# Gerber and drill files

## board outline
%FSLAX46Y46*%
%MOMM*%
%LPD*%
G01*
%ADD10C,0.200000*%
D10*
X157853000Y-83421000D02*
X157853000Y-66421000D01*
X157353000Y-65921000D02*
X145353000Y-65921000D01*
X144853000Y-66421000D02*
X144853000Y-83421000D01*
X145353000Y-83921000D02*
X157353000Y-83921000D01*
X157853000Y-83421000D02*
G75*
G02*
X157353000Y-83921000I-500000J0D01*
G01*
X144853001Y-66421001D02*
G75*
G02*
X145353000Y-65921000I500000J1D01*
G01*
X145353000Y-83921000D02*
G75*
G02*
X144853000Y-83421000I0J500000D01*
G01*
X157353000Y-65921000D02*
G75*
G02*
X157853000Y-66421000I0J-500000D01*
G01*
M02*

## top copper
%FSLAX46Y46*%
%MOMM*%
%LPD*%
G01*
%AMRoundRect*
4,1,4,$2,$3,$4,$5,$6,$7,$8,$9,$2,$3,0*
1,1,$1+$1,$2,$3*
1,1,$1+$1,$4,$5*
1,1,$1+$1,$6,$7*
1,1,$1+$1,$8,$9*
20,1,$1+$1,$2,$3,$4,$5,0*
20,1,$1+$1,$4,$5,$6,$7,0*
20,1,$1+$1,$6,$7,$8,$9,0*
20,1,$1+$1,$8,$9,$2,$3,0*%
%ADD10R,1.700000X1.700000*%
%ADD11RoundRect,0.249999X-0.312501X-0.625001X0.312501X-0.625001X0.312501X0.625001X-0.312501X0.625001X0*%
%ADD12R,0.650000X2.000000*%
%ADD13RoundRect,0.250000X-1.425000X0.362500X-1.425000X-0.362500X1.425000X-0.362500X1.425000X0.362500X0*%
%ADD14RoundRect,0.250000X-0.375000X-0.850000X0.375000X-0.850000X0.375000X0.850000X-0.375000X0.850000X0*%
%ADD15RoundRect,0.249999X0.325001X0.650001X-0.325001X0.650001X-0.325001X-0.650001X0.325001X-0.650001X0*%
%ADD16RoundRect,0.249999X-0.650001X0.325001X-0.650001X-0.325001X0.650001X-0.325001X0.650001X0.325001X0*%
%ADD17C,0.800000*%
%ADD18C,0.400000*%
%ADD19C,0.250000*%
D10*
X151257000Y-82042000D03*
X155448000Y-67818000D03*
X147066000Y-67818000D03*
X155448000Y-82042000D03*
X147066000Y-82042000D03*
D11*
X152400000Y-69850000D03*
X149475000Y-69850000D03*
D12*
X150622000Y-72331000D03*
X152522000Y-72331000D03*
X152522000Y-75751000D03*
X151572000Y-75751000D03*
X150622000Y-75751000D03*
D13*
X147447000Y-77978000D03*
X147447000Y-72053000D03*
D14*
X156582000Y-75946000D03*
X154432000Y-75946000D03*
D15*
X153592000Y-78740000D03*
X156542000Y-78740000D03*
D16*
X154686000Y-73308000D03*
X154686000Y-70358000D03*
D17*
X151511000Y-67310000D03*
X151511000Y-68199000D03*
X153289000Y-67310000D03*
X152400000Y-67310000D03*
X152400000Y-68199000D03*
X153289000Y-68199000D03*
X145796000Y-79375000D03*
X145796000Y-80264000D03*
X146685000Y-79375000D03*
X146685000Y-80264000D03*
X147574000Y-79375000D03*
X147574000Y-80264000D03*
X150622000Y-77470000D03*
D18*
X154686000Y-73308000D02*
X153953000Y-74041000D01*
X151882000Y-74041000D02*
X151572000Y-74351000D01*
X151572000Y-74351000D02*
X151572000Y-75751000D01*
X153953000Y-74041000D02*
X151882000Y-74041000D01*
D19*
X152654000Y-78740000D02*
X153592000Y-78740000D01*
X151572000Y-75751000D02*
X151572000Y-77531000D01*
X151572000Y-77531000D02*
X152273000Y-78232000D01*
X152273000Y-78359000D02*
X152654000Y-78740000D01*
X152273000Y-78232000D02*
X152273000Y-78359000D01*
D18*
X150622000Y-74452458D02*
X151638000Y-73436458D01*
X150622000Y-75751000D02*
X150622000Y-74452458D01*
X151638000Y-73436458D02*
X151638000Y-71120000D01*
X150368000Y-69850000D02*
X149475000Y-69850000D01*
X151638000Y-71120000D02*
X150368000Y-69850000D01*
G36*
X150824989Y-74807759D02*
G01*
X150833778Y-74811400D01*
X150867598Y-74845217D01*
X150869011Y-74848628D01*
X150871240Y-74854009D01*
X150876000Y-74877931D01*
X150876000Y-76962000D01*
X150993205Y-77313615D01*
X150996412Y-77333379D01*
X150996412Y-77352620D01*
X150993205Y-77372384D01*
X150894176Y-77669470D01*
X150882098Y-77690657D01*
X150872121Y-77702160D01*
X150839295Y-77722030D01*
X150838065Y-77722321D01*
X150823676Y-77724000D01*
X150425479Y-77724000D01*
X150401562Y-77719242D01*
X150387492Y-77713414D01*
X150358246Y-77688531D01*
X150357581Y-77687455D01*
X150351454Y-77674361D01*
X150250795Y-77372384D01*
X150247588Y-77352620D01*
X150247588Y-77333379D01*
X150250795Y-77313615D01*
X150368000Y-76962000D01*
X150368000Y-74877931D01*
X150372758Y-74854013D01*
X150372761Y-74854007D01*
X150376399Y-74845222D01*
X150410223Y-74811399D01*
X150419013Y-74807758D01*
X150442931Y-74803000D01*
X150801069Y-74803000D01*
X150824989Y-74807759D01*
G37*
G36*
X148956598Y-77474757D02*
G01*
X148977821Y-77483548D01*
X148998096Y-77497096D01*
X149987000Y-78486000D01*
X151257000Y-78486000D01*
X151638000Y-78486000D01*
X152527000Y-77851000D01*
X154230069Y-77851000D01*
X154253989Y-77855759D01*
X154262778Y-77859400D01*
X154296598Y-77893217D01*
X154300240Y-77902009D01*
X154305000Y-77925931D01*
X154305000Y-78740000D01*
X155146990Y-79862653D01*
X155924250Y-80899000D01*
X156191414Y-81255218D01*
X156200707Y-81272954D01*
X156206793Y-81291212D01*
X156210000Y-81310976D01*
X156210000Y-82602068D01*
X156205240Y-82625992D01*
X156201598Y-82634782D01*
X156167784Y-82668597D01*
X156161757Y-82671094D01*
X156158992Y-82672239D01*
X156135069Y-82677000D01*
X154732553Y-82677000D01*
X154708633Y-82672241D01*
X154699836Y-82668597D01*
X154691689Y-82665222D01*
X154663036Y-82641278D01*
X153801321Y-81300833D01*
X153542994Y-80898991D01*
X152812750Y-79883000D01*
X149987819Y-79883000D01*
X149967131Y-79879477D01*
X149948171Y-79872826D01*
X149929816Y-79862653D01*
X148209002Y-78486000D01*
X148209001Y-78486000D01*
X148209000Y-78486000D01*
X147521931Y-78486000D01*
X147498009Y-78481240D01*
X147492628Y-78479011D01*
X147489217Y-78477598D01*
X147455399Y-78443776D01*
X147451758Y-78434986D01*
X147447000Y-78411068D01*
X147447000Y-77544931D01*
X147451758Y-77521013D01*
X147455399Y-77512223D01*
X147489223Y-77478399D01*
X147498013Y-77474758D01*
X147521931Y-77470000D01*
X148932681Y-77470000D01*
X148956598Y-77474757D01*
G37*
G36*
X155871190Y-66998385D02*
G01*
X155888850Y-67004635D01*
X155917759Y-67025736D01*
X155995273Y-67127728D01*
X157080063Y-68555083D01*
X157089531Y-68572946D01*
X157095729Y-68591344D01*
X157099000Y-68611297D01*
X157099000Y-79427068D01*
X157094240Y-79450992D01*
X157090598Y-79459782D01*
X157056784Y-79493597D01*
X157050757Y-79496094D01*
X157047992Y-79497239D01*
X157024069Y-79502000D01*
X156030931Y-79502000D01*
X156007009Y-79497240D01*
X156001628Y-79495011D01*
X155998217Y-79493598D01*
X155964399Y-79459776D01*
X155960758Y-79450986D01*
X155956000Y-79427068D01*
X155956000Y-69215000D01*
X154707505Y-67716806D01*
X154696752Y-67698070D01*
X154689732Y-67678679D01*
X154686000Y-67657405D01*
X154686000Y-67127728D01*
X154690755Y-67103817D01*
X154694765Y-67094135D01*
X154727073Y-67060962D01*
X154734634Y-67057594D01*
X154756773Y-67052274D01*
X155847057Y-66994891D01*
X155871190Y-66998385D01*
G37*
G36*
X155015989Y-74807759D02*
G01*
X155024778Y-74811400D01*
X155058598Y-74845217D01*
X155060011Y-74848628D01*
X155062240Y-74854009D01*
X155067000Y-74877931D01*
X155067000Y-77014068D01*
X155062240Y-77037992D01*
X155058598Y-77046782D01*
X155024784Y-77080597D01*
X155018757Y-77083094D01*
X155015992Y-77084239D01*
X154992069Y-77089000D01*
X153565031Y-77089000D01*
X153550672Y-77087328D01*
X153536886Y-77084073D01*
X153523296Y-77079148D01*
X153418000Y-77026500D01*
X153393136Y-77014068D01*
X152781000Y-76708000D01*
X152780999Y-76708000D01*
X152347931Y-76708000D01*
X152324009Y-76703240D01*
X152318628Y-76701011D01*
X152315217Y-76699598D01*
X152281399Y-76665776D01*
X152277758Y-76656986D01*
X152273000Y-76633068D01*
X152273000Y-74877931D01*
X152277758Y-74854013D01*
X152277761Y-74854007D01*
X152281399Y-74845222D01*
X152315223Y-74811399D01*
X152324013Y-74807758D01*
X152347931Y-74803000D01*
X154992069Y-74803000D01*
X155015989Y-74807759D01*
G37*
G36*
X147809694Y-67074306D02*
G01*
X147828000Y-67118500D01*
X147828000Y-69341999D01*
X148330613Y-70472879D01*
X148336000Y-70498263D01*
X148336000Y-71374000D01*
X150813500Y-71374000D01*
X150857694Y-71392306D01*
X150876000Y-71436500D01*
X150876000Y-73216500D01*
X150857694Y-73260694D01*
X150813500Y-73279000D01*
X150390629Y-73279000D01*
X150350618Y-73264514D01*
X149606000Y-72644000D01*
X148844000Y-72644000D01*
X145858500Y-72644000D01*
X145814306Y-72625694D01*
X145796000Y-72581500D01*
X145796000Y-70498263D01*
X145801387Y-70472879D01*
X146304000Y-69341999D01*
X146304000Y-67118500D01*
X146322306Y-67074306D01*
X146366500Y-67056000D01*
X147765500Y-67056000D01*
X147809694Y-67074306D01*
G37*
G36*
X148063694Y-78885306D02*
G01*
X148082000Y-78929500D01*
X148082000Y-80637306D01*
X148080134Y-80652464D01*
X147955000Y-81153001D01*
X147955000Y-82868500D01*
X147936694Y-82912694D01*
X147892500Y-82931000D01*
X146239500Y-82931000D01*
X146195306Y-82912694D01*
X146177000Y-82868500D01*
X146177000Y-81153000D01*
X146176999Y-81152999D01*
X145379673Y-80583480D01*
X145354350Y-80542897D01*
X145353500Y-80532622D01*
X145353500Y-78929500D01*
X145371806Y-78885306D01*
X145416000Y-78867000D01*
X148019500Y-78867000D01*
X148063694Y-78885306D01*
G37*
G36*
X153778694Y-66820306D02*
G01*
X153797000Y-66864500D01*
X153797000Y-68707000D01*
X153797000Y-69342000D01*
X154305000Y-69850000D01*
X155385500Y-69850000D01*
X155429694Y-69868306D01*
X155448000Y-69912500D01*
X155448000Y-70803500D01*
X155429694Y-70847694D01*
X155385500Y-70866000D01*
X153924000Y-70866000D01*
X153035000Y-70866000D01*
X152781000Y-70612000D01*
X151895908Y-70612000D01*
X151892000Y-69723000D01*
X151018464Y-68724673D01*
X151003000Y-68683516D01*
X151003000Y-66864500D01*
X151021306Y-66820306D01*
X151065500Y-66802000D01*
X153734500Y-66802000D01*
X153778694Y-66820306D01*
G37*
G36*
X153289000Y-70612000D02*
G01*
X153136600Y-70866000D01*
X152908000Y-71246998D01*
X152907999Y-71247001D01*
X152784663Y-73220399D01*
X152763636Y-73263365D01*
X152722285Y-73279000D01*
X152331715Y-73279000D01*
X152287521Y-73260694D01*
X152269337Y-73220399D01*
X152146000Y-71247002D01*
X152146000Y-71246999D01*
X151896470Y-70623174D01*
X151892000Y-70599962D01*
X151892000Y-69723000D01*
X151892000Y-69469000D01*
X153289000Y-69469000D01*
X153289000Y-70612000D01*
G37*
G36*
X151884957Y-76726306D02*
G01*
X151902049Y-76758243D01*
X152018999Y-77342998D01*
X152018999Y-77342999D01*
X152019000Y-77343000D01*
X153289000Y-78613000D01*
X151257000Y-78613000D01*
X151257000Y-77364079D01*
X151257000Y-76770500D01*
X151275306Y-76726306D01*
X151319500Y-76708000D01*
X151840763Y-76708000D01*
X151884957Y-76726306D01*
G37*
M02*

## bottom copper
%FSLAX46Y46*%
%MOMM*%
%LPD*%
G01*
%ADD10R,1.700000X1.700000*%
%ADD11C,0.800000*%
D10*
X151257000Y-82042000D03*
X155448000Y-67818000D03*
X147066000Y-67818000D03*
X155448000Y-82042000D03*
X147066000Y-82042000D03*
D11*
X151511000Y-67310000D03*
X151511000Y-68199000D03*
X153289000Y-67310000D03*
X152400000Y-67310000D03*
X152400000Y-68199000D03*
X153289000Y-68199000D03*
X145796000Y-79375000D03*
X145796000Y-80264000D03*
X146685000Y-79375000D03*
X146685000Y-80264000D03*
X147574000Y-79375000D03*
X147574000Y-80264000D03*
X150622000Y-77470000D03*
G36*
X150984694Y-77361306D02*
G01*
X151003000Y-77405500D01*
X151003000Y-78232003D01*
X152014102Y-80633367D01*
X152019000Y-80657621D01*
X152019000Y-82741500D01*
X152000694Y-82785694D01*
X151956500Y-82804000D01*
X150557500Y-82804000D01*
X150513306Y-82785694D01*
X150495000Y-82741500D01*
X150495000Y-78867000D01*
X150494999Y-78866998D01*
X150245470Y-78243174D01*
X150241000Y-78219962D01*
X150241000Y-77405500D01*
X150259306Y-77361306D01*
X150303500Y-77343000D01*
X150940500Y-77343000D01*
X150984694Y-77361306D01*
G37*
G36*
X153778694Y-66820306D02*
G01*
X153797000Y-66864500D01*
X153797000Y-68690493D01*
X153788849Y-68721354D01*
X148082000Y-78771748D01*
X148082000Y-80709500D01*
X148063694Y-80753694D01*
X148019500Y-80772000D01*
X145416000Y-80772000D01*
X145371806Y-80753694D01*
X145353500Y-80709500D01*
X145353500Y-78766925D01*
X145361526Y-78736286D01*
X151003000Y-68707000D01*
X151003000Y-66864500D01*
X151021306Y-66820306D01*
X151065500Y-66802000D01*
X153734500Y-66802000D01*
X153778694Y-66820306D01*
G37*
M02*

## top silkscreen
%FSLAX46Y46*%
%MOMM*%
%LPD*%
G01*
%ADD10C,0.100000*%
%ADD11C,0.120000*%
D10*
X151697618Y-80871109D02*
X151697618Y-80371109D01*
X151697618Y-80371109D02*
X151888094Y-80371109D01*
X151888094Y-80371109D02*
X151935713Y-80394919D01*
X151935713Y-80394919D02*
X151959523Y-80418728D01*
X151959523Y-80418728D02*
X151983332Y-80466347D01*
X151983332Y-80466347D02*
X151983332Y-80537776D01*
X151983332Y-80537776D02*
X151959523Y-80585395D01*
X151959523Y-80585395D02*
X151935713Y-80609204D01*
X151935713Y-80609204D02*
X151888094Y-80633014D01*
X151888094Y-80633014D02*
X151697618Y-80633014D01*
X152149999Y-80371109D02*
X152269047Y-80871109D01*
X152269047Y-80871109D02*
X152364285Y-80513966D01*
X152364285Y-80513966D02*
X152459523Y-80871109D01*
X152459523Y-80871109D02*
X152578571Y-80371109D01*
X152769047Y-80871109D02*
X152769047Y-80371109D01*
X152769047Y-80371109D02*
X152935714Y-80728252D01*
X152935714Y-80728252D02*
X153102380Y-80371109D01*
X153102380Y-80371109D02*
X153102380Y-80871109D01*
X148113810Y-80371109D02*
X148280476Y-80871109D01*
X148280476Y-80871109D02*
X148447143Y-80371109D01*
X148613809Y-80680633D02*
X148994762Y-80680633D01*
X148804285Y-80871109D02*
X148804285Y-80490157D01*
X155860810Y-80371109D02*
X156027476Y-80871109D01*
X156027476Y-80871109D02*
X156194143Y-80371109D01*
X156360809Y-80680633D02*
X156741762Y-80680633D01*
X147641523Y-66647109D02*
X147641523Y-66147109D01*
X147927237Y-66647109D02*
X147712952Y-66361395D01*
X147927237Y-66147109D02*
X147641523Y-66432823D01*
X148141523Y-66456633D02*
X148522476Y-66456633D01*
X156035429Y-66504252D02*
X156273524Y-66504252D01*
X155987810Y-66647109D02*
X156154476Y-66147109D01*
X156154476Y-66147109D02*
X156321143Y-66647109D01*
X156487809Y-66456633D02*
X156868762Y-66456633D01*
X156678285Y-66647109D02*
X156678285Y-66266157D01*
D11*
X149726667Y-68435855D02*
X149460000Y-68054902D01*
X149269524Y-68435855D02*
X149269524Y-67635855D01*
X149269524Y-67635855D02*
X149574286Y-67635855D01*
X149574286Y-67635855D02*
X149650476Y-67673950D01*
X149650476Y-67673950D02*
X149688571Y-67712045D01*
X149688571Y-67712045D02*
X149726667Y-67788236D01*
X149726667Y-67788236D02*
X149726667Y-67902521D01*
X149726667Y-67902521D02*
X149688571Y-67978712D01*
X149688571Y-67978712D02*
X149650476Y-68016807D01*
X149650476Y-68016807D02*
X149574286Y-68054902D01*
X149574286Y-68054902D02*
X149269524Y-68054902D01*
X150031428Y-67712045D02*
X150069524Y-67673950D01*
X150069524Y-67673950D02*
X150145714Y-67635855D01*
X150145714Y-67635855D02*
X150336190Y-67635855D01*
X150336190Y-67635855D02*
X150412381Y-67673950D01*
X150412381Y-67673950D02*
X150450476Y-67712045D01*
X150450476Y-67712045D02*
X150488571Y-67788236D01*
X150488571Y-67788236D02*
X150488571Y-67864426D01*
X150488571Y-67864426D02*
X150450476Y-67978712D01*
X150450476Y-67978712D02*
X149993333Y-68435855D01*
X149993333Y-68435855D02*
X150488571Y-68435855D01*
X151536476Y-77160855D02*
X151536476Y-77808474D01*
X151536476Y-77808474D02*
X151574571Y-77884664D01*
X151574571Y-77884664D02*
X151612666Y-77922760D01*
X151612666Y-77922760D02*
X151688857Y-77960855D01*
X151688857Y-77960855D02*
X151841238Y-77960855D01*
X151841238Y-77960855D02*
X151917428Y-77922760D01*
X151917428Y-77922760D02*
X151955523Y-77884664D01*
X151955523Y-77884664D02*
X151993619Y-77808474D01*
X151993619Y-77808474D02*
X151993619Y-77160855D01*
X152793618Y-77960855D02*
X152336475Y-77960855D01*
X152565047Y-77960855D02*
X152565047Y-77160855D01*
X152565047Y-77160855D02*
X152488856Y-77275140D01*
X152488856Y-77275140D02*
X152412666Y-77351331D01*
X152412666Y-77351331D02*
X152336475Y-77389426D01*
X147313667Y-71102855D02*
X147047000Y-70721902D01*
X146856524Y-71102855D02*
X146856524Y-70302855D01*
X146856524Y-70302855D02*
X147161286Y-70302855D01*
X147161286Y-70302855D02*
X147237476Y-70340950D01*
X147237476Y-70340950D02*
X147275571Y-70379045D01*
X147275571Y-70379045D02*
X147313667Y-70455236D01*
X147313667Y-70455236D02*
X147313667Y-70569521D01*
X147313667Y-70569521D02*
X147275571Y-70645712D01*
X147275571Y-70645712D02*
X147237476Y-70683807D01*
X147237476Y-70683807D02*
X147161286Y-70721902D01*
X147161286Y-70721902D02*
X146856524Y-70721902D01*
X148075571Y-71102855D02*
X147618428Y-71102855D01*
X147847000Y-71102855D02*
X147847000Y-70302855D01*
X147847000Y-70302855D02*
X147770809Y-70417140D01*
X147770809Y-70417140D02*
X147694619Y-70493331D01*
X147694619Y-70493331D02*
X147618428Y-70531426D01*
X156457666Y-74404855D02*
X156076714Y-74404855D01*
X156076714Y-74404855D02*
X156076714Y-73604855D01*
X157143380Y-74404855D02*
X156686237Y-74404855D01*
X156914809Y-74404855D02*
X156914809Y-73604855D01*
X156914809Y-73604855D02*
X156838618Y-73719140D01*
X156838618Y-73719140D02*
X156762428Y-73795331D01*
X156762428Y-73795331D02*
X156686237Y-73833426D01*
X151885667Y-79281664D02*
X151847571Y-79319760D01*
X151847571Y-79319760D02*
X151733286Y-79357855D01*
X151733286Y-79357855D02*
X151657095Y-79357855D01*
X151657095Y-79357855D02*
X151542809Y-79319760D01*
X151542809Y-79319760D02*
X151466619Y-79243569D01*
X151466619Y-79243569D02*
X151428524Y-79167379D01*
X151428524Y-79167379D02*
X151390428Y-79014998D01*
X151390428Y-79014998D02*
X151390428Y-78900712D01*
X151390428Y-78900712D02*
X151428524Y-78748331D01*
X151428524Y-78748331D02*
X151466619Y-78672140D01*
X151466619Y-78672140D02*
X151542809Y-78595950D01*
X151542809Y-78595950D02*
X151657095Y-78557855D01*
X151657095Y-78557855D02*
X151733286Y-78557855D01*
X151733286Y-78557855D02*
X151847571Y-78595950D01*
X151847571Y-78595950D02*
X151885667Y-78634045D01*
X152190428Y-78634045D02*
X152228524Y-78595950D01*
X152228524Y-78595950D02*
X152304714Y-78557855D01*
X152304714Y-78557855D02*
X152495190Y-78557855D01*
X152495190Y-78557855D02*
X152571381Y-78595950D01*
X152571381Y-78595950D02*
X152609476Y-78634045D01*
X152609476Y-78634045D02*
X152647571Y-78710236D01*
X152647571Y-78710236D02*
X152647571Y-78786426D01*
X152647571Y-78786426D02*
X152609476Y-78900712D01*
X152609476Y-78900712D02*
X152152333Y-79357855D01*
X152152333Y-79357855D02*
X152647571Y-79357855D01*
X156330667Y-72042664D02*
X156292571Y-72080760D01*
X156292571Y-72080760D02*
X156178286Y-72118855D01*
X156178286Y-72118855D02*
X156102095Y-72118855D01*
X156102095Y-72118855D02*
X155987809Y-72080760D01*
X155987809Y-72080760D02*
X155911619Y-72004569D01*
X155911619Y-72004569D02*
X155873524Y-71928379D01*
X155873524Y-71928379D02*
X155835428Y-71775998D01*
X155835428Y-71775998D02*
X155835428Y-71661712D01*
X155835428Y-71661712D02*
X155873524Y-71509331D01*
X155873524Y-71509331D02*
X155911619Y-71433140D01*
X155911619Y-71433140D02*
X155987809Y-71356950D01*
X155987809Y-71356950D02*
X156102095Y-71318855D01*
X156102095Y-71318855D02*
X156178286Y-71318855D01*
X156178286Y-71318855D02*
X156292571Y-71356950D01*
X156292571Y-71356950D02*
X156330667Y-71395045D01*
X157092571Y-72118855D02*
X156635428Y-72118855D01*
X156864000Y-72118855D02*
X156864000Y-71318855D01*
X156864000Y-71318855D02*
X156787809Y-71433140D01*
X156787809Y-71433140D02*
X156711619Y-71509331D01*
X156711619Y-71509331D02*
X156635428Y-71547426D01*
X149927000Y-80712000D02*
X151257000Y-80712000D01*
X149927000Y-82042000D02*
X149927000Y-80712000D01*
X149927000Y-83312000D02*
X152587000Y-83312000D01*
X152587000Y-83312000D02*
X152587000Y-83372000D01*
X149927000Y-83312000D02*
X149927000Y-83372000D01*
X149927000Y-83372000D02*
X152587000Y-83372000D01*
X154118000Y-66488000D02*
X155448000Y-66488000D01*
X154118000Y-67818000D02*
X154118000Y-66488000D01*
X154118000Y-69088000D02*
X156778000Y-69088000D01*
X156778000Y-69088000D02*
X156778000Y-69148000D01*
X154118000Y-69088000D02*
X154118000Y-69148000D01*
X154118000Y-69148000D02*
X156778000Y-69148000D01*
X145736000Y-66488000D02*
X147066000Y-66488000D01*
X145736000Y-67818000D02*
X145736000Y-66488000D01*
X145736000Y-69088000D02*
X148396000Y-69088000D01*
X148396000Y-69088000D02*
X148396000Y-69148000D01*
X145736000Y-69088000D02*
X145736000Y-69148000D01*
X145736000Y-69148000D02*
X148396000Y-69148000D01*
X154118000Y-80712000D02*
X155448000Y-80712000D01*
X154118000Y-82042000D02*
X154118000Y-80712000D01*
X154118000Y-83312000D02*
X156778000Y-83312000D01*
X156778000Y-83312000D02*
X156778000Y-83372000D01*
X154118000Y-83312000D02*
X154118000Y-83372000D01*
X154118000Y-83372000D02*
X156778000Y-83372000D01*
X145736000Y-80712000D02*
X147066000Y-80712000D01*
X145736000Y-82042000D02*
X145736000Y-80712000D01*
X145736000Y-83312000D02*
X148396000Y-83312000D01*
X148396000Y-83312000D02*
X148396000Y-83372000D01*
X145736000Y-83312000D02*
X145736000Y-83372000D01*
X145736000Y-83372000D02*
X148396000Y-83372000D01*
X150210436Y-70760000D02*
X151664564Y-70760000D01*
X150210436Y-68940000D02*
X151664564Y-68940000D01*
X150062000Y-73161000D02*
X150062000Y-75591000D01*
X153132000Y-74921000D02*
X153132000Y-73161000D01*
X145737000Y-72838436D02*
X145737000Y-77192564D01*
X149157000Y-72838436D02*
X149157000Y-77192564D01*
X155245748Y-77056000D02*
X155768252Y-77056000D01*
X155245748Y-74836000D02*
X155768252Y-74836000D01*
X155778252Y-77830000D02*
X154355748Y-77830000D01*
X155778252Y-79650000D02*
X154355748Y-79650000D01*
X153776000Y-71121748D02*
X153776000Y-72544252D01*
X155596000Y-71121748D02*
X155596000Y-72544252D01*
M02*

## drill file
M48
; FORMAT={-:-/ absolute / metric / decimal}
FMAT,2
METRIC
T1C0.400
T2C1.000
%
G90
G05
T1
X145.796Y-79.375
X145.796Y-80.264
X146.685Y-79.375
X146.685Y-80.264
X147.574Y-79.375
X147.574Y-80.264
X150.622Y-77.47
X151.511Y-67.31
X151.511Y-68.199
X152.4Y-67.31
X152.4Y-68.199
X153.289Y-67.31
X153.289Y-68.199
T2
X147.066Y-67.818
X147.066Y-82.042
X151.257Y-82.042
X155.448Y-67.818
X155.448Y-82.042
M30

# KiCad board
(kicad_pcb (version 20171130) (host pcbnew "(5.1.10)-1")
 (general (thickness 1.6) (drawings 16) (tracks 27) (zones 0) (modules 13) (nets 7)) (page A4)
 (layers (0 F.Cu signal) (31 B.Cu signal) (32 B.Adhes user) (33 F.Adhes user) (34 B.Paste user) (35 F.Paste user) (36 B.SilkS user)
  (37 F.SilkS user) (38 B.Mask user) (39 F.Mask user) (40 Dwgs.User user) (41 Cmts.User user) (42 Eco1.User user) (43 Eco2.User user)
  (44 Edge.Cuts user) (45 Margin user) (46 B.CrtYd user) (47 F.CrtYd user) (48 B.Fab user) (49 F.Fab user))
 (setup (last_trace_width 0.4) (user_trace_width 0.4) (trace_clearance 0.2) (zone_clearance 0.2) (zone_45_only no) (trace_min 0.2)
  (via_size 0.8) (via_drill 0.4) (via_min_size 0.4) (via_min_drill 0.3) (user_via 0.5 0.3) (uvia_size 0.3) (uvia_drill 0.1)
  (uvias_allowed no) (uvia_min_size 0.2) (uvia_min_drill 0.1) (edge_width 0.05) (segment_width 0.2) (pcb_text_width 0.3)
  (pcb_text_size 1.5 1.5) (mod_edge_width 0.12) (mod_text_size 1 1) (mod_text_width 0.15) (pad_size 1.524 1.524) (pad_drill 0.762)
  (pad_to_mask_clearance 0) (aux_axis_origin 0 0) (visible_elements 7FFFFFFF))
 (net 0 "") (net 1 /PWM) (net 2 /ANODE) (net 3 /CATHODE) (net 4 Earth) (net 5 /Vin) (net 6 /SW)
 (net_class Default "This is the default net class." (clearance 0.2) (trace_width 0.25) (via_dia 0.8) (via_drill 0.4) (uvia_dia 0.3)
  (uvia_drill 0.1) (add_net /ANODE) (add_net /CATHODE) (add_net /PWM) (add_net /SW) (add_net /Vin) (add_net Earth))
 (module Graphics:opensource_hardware (layer B.Cu) (at 146.558 70.993 180)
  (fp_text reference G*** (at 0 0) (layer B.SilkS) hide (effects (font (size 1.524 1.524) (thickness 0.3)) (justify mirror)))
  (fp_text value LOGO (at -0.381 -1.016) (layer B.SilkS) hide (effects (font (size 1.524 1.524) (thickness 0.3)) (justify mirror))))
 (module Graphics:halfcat (layer B.Cu) (at 148.971 71.247 180)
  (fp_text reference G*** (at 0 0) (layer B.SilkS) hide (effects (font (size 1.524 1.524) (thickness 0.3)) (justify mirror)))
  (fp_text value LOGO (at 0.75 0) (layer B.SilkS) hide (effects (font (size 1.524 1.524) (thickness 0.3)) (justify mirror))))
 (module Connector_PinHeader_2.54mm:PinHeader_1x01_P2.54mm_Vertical (layer F.Cu) (at 151.257 82.042)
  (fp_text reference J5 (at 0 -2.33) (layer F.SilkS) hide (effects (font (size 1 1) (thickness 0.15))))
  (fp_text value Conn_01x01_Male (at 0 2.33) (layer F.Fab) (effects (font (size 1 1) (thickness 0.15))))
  (fp_line (start -1.33 -1.33) (end 0 -1.33) (layer F.SilkS) (width 0.12))
  (fp_line (start -1.33 0) (end -1.33 -1.33) (layer F.SilkS) (width 0.12))
  (fp_line (start -1.33 1.27) (end 1.33 1.27) (layer F.SilkS) (width 0.12))
  (fp_line (start 1.33 1.27) (end 1.33 1.33) (layer F.SilkS) (width 0.12))
  (fp_line (start -1.33 1.27) (end -1.33 1.33) (layer F.SilkS) (width 0.12))
  (fp_line (start -1.33 1.33) (end 1.33 1.33) (layer F.SilkS) (width 0.12))
  (pad 1 thru_hole rect (at 0 0) (size 1.7 1.7) (drill 1) (layers *.Cu *.Mask) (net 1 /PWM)))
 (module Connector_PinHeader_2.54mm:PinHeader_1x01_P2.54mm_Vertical (layer F.Cu) (at 155.448 67.818)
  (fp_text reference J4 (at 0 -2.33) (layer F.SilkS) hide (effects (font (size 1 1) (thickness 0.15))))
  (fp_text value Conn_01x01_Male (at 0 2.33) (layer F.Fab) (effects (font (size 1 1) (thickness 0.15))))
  (fp_line (start -1.33 -1.33) (end 0 -1.33) (layer F.SilkS) (width 0.12))
  (fp_line (start -1.33 0) (end -1.33 -1.33) (layer F.SilkS) (width 0.12))
  (fp_line (start -1.33 1.27) (end 1.33 1.27) (layer F.SilkS) (width 0.12))
  (fp_line (start 1.33 1.27) (end 1.33 1.33) (layer F.SilkS) (width 0.12))
  (fp_line (start -1.33 1.27) (end -1.33 1.33) (layer F.SilkS) (width 0.12))
  (fp_line (start -1.33 1.33) (end 1.33 1.33) (layer F.SilkS) (width 0.12))
  (pad 1 thru_hole rect (at 0 0) (size 1.7 1.7) (drill 1) (layers *.Cu *.Mask) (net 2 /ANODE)))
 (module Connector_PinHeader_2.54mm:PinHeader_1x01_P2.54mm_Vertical (layer F.Cu) (at 147.066 67.818)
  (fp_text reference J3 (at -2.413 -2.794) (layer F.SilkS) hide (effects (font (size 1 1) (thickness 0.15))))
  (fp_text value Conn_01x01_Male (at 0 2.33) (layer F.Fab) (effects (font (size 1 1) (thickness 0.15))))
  (fp_line (start -1.33 -1.33) (end 0 -1.33) (layer F.SilkS) (width 0.12))
  (fp_line (start -1.33 0) (end -1.33 -1.33) (layer F.SilkS) (width 0.12))
  (fp_line (start -1.33 1.27) (end 1.33 1.27) (layer F.SilkS) (width 0.12))
  (fp_line (start 1.33 1.27) (end 1.33 1.33) (layer F.SilkS) (width 0.12))
  (fp_line (start -1.33 1.27) (end -1.33 1.33) (layer F.SilkS) (width 0.12))
  (fp_line (start -1.33 1.33) (end 1.33 1.33) (layer F.SilkS) (width 0.12))
  (pad 1 thru_hole rect (at 0 0) (size 1.7 1.7) (drill 1) (layers *.Cu *.Mask) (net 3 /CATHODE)))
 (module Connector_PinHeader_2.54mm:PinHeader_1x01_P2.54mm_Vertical (layer F.Cu) (at 155.448 82.042)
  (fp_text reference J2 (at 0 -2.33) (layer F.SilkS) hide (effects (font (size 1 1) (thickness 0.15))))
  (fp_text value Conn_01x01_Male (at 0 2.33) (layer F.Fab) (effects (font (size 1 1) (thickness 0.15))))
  (fp_line (start -1.33 -1.33) (end 0 -1.33) (layer F.SilkS) (width 0.12))
  (fp_line (start -1.33 0) (end -1.33 -1.33) (layer F.SilkS) (width 0.12))
  (fp_line (start -1.33 1.27) (end 1.33 1.27) (layer F.SilkS) (width 0.12))
  (fp_line (start 1.33 1.27) (end 1.33 1.33) (layer F.SilkS) (width 0.12))
  (fp_line (start -1.33 1.27) (end -1.33 1.33) (layer F.SilkS) (width 0.12))
  (fp_line (start -1.33 1.33) (end 1.33 1.33) (layer F.SilkS) (width 0.12))
  (pad 1 thru_hole rect (at 0 0) (size 1.7 1.7) (drill 1) (layers *.Cu *.Mask) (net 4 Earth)))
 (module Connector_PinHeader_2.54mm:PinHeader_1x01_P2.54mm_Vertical (layer F.Cu) (at 147.066 82.042)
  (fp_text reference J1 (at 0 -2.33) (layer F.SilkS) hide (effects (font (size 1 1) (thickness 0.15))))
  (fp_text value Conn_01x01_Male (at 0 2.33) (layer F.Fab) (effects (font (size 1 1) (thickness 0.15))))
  (fp_line (start -1.33 -1.33) (end 0 -1.33) (layer F.SilkS) (width 0.12))
  (fp_line (start -1.33 0) (end -1.33 -1.33) (layer F.SilkS) (width 0.12))
  (fp_line (start -1.33 1.27) (end 1.33 1.27) (layer F.SilkS) (width 0.12))
  (fp_line (start 1.33 1.27) (end 1.33 1.33) (layer F.SilkS) (width 0.12))
  (fp_line (start -1.33 1.27) (end -1.33 1.33) (layer F.SilkS) (width 0.12))
  (fp_line (start -1.33 1.33) (end 1.33 1.33) (layer F.SilkS) (width 0.12))
  (pad 1 thru_hole rect (at 0 0) (size 1.7 1.7) (drill 1) (layers *.Cu *.Mask) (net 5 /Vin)))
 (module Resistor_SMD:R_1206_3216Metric (layer F.Cu) (at 150.9375 69.85)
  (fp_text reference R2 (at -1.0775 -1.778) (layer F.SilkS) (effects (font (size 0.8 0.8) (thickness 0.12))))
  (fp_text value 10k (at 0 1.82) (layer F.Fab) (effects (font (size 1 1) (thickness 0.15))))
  (fp_line (start -0.727064 0.91) (end 0.727064 0.91) (layer F.SilkS) (width 0.12))
  (fp_line (start -0.727064 -0.91) (end 0.727064 -0.91) (layer F.SilkS) (width 0.12))
  (pad 2 smd roundrect (at 1.4625 0) (size 1.125 1.75) (layers F.Cu F.Paste F.Mask) (roundrect_rratio 0.2222213333333333) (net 5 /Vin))
  (pad 1 smd roundrect (at -1.4625 0) (size 1.125 1.75) (layers F.Cu F.Paste F.Mask) (roundrect_rratio 0.2222213333333333) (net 1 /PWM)))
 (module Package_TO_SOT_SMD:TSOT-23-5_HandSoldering (layer F.Cu) (at 151.572 74.041 90)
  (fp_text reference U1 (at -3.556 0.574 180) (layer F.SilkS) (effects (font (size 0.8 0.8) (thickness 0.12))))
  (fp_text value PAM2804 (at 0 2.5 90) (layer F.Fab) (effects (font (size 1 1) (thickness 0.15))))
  (fp_line (start 0.88 -1.51) (end -1.55 -1.51) (layer F.SilkS) (width 0.12))
  (fp_line (start -0.88 1.56) (end 0.88 1.56) (layer F.SilkS) (width 0.12))
  (pad 5 smd rect (at 1.71 -0.95 90) (size 2 0.65) (layers F.Cu F.Paste F.Mask) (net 3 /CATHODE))
  (pad 4 smd rect (at 1.71 0.95 90) (size 2 0.65) (layers F.Cu F.Paste F.Mask) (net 5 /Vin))
  (pad 3 smd rect (at -1.71 0.95 90) (size 2 0.65) (layers F.Cu F.Paste F.Mask) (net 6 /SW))
  (pad 2 smd rect (at -1.71 0 90) (size 2 0.65) (layers F.Cu F.Paste F.Mask) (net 4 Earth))
  (pad 1 smd rect (at -1.71 -0.95 90) (size 2 0.65) (layers F.Cu F.Paste F.Mask) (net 1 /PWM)))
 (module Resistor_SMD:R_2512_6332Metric (layer F.Cu) (at 147.447 75.0155 270)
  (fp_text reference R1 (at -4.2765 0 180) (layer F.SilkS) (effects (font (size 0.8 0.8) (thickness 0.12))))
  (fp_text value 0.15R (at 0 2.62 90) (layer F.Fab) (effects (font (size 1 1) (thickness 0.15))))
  (fp_line (start -2.177064 1.71) (end 2.177064 1.71) (layer F.SilkS) (width 0.12))
  (fp_line (start -2.177064 -1.71) (end 2.177064 -1.71) (layer F.SilkS) (width 0.12))
  (pad 2 smd roundrect (at 2.9625 0 270) (size 1.225 3.35) (layers F.Cu F.Paste F.Mask) (roundrect_rratio 0.2040816326530612) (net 4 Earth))
  (pad 1 smd roundrect (at -2.9625 0 270) (size 1.225 3.35) (layers F.Cu F.Paste F.Mask) (roundrect_rratio 0.2040816326530612)
   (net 3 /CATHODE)))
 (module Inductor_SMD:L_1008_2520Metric (layer F.Cu) (at 155.507 75.946)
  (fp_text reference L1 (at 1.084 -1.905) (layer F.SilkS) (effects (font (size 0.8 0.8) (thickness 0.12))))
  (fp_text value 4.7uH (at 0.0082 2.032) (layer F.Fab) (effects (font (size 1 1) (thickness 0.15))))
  (fp_line (start -0.261252 1.11) (end 0.261252 1.11) (layer F.SilkS) (width 0.12))
  (fp_line (start -0.261252 -1.11) (end 0.261252 -1.11) (layer F.SilkS) (width 0.12))
  (pad 2 smd roundrect (at 1.075 0) (size 1.25 2.2) (layers F.Cu F.Paste F.Mask) (roundrect_rratio 0.2) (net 2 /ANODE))
  (pad 1 smd roundrect (at -1.075 0) (size 1.25 2.2) (layers F.Cu F.Paste F.Mask) (roundrect_rratio 0.2) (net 6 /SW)))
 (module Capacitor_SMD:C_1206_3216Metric (layer F.Cu) (at 155.067 78.74 180)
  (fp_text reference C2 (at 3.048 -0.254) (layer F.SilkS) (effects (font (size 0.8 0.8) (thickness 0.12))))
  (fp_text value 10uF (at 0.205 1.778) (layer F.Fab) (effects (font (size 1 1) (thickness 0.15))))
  (fp_line (start -0.711252 0.91) (end 0.711252 0.91) (layer F.SilkS) (width 0.12))
  (fp_line (start -0.711252 -0.91) (end 0.711252 -0.91) (layer F.SilkS) (width 0.12))
  (pad 2 smd roundrect (at 1.475 0 180) (size 1.15 1.8) (layers F.Cu F.Paste F.Mask) (roundrect_rratio 0.2173904347826087) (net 4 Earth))
  (pad 1 smd roundrect (at -1.475 0 180) (size 1.15 1.8) (layers F.Cu F.Paste F.Mask) (roundrect_rratio 0.2173904347826087) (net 2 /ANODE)))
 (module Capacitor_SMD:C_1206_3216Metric (layer F.Cu) (at 154.686 71.833 270)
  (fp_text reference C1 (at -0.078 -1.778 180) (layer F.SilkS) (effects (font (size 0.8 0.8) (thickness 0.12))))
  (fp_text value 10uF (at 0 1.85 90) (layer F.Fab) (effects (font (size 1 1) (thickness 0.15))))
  (fp_line (start -0.711252 0.91) (end 0.711252 0.91) (layer F.SilkS) (width 0.12))
  (fp_line (start -0.711252 -0.91) (end 0.711252 -0.91) (layer F.SilkS) (width 0.12))
  (pad 2 smd roundrect (at 1.475 0 270) (size 1.15 1.8) (layers F.Cu F.Paste F.Mask) (roundrect_rratio 0.2173904347826087) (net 4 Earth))
  (pad 1 smd roundrect (at -1.475 0 270) (size 1.15 1.8) (layers F.Cu F.Paste F.Mask) (roundrect_rratio 0.2173904347826087) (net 5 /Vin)))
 (gr_line (start 157.853 83.421) (end 157.853 66.421) (layer Edge.Cuts) (width 0.2))
 (gr_line (start 157.353 65.921) (end 145.353 65.921) (layer Edge.Cuts) (width 0.2))
 (gr_line (start 144.853 66.421) (end 144.853 83.421) (layer Edge.Cuts) (width 0.2))
 (gr_line (start 145.353 83.921) (end 157.353 83.921) (layer Edge.Cuts) (width 0.2))
 (gr_arc (start 157.353 83.421) (end 157.353 83.921) (angle -90) (layer Edge.Cuts) (width 0.2))
 (gr_arc (start 145.353001 66.421) (end 145.353 65.921) (angle -90) (layer Edge.Cuts) (width 0.2))
 (gr_arc (start 145.353 83.421) (end 144.853 83.421) (angle -90) (layer Edge.Cuts) (width 0.2))
 (gr_arc (start 157.353 66.421) (end 157.853 66.421) (angle -90) (layer Edge.Cuts) (width 0.2))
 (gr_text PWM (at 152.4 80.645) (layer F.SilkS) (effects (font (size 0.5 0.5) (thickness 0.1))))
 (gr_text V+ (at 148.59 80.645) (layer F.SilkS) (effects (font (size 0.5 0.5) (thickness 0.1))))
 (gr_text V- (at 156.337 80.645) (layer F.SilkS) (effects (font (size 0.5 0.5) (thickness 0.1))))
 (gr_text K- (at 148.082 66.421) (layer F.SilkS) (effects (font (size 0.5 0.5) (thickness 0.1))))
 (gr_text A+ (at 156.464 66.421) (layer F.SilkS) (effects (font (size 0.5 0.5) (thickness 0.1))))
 (via (at 151.511 67.31) (size 0.8) (drill 0.4) (layers F.Cu B.Cu) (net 5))
 (via (at 151.511 68.199) (size 0.8) (drill 0.4) (layers F.Cu B.Cu) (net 5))
 (segment (start 154.686 73.308) (end 153.953 74.041) (width 0.4) (layer F.Cu) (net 4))
 (segment (start 151.882 74.041) (end 151.572 74.351) (width 0.4) (layer F.Cu) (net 4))
 (segment (start 151.572 74.351) (end 151.572 75.751) (width 0.4) (layer F.Cu) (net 4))
 (segment (start 153.953 74.041) (end 151.882 74.041) (width 0.4) (layer F.Cu) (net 4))
 (segment (start 152.654 78.74) (end 153.592 78.74) (width 0.25) (layer F.Cu) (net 4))
 (segment (start 151.572 75.751) (end 151.572 77.531) (width 0.25) (layer F.Cu) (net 4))
 (segment (start 151.572 77.531) (end 152.273 78.232) (width 0.25) (layer F.Cu) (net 4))
 (segment (start 152.273 78.359) (end 152.654 78.74) (width 0.25) (layer F.Cu) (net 4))
 (segment (start 152.273 78.232) (end 152.273 78.359) (width 0.25) (layer F.Cu) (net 4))
 (via (at 153.289 67.31) (size 0.8) (drill 0.4) (layers F.Cu B.Cu) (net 5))
 (via (at 152.4 67.31) (size 0.8) (drill 0.4) (layers F.Cu B.Cu) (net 5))
 (via (at 152.4 68.199) (size 0.8) (drill 0.4) (layers F.Cu B.Cu) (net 5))
 (via (at 153.289 68.199) (size 0.8) (drill 0.4) (layers F.Cu B.Cu) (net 5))
 (via (at 145.796 79.375) (size 0.8) (drill 0.4) (layers F.Cu B.Cu) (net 5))
 (via (at 145.796 80.264) (size 0.8) (drill 0.4) (layers F.Cu B.Cu) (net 5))
 (via (at 146.685 79.375) (size 0.8) (drill 0.4) (layers F.Cu B.Cu) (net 5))
 (via (at 146.685 80.264) (size 0.8) (drill 0.4) (layers F.Cu B.Cu) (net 5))
 (via (at 147.574 79.375) (size 0.8) (drill 0.4) (layers F.Cu B.Cu) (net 5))
 (via (at 147.574 80.264) (size 0.8) (drill 0.4) (layers F.Cu B.Cu) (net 5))
 (via (at 150.622 77.47) (size 0.8) (drill 0.4) (layers F.Cu B.Cu) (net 1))
 (segment (start 150.622 74.452458) (end 151.638 73.436458) (width 0.4) (layer F.Cu) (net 1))
 (segment (start 150.622 75.751) (end 150.622 74.452458) (width 0.4) (layer F.Cu) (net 1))
 (segment (start 151.638 73.436458) (end 151.638 71.12) (width 0.4) (layer F.Cu) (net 1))
 (segment (start 150.368 69.85) (end 149.475 69.85) (width 0.4) (layer F.Cu) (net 1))
 (segment (start 151.638 71.12) (end 150.368 69.85) (width 0.4) (layer F.Cu) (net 1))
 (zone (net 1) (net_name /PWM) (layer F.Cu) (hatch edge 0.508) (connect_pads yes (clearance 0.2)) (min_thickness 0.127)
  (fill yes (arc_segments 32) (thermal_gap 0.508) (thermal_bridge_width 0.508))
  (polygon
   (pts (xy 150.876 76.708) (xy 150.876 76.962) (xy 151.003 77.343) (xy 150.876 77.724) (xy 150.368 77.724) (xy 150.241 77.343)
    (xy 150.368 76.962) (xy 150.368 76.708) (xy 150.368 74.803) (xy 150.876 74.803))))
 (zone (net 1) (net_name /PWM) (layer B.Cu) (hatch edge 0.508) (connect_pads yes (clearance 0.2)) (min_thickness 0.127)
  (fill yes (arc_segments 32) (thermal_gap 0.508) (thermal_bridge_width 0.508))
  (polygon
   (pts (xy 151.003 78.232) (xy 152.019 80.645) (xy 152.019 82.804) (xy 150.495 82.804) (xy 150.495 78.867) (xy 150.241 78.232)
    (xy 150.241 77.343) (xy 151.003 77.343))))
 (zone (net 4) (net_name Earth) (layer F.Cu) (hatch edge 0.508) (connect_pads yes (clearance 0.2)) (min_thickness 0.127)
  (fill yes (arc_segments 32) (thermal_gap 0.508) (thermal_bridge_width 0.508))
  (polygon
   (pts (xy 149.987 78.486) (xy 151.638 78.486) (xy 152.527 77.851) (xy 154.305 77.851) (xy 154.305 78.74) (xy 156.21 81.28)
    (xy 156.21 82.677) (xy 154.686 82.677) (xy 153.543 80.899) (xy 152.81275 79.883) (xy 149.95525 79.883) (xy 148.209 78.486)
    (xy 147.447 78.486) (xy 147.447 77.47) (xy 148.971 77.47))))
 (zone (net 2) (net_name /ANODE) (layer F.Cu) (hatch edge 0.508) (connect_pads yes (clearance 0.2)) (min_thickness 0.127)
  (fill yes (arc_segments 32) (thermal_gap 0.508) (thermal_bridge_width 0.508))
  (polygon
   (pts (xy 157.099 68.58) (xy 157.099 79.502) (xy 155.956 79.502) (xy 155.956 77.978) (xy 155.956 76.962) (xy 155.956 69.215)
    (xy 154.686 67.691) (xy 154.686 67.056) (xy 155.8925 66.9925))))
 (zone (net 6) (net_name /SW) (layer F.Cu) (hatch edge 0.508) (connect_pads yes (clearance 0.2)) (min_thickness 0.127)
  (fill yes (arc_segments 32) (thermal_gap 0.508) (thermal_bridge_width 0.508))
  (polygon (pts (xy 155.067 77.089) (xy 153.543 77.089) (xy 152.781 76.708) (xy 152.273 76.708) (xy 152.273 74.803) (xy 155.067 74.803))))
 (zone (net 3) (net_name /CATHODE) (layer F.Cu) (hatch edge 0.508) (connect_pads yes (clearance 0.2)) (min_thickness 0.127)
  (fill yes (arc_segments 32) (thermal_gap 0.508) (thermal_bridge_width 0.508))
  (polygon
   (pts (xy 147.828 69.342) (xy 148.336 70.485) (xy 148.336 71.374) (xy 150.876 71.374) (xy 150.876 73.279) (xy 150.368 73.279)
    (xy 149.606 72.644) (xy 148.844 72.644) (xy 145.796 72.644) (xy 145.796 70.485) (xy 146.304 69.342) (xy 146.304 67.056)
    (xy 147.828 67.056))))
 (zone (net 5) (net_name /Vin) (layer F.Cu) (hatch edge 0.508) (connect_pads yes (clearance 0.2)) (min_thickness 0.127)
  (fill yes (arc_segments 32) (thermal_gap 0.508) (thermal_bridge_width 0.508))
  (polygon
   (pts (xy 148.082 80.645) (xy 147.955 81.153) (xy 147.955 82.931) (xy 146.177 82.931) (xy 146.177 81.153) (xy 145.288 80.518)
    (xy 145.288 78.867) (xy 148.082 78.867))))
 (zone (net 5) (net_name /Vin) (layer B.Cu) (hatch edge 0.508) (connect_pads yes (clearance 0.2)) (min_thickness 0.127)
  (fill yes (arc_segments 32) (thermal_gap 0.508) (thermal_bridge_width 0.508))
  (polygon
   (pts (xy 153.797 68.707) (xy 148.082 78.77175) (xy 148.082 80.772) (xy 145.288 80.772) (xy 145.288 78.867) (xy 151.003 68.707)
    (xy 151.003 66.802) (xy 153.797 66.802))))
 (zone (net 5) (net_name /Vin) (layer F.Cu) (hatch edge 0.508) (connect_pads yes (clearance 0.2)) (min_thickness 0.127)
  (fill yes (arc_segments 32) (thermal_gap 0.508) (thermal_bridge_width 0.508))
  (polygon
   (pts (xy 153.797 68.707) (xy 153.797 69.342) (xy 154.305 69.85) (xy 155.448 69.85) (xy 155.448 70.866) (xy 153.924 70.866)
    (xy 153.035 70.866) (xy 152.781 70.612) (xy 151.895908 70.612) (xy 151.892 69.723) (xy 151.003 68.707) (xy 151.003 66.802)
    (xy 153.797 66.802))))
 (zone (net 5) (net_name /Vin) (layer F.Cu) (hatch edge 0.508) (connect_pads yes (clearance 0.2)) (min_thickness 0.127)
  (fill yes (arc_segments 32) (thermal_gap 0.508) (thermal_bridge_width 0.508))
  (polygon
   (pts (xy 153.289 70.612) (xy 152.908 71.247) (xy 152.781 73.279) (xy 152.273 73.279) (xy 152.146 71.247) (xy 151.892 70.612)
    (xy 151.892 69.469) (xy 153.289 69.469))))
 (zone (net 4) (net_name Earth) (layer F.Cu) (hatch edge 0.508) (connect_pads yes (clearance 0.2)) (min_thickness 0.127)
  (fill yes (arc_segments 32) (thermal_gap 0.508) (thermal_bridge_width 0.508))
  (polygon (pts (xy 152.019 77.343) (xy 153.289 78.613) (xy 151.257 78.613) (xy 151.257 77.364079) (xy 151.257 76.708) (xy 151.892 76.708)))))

